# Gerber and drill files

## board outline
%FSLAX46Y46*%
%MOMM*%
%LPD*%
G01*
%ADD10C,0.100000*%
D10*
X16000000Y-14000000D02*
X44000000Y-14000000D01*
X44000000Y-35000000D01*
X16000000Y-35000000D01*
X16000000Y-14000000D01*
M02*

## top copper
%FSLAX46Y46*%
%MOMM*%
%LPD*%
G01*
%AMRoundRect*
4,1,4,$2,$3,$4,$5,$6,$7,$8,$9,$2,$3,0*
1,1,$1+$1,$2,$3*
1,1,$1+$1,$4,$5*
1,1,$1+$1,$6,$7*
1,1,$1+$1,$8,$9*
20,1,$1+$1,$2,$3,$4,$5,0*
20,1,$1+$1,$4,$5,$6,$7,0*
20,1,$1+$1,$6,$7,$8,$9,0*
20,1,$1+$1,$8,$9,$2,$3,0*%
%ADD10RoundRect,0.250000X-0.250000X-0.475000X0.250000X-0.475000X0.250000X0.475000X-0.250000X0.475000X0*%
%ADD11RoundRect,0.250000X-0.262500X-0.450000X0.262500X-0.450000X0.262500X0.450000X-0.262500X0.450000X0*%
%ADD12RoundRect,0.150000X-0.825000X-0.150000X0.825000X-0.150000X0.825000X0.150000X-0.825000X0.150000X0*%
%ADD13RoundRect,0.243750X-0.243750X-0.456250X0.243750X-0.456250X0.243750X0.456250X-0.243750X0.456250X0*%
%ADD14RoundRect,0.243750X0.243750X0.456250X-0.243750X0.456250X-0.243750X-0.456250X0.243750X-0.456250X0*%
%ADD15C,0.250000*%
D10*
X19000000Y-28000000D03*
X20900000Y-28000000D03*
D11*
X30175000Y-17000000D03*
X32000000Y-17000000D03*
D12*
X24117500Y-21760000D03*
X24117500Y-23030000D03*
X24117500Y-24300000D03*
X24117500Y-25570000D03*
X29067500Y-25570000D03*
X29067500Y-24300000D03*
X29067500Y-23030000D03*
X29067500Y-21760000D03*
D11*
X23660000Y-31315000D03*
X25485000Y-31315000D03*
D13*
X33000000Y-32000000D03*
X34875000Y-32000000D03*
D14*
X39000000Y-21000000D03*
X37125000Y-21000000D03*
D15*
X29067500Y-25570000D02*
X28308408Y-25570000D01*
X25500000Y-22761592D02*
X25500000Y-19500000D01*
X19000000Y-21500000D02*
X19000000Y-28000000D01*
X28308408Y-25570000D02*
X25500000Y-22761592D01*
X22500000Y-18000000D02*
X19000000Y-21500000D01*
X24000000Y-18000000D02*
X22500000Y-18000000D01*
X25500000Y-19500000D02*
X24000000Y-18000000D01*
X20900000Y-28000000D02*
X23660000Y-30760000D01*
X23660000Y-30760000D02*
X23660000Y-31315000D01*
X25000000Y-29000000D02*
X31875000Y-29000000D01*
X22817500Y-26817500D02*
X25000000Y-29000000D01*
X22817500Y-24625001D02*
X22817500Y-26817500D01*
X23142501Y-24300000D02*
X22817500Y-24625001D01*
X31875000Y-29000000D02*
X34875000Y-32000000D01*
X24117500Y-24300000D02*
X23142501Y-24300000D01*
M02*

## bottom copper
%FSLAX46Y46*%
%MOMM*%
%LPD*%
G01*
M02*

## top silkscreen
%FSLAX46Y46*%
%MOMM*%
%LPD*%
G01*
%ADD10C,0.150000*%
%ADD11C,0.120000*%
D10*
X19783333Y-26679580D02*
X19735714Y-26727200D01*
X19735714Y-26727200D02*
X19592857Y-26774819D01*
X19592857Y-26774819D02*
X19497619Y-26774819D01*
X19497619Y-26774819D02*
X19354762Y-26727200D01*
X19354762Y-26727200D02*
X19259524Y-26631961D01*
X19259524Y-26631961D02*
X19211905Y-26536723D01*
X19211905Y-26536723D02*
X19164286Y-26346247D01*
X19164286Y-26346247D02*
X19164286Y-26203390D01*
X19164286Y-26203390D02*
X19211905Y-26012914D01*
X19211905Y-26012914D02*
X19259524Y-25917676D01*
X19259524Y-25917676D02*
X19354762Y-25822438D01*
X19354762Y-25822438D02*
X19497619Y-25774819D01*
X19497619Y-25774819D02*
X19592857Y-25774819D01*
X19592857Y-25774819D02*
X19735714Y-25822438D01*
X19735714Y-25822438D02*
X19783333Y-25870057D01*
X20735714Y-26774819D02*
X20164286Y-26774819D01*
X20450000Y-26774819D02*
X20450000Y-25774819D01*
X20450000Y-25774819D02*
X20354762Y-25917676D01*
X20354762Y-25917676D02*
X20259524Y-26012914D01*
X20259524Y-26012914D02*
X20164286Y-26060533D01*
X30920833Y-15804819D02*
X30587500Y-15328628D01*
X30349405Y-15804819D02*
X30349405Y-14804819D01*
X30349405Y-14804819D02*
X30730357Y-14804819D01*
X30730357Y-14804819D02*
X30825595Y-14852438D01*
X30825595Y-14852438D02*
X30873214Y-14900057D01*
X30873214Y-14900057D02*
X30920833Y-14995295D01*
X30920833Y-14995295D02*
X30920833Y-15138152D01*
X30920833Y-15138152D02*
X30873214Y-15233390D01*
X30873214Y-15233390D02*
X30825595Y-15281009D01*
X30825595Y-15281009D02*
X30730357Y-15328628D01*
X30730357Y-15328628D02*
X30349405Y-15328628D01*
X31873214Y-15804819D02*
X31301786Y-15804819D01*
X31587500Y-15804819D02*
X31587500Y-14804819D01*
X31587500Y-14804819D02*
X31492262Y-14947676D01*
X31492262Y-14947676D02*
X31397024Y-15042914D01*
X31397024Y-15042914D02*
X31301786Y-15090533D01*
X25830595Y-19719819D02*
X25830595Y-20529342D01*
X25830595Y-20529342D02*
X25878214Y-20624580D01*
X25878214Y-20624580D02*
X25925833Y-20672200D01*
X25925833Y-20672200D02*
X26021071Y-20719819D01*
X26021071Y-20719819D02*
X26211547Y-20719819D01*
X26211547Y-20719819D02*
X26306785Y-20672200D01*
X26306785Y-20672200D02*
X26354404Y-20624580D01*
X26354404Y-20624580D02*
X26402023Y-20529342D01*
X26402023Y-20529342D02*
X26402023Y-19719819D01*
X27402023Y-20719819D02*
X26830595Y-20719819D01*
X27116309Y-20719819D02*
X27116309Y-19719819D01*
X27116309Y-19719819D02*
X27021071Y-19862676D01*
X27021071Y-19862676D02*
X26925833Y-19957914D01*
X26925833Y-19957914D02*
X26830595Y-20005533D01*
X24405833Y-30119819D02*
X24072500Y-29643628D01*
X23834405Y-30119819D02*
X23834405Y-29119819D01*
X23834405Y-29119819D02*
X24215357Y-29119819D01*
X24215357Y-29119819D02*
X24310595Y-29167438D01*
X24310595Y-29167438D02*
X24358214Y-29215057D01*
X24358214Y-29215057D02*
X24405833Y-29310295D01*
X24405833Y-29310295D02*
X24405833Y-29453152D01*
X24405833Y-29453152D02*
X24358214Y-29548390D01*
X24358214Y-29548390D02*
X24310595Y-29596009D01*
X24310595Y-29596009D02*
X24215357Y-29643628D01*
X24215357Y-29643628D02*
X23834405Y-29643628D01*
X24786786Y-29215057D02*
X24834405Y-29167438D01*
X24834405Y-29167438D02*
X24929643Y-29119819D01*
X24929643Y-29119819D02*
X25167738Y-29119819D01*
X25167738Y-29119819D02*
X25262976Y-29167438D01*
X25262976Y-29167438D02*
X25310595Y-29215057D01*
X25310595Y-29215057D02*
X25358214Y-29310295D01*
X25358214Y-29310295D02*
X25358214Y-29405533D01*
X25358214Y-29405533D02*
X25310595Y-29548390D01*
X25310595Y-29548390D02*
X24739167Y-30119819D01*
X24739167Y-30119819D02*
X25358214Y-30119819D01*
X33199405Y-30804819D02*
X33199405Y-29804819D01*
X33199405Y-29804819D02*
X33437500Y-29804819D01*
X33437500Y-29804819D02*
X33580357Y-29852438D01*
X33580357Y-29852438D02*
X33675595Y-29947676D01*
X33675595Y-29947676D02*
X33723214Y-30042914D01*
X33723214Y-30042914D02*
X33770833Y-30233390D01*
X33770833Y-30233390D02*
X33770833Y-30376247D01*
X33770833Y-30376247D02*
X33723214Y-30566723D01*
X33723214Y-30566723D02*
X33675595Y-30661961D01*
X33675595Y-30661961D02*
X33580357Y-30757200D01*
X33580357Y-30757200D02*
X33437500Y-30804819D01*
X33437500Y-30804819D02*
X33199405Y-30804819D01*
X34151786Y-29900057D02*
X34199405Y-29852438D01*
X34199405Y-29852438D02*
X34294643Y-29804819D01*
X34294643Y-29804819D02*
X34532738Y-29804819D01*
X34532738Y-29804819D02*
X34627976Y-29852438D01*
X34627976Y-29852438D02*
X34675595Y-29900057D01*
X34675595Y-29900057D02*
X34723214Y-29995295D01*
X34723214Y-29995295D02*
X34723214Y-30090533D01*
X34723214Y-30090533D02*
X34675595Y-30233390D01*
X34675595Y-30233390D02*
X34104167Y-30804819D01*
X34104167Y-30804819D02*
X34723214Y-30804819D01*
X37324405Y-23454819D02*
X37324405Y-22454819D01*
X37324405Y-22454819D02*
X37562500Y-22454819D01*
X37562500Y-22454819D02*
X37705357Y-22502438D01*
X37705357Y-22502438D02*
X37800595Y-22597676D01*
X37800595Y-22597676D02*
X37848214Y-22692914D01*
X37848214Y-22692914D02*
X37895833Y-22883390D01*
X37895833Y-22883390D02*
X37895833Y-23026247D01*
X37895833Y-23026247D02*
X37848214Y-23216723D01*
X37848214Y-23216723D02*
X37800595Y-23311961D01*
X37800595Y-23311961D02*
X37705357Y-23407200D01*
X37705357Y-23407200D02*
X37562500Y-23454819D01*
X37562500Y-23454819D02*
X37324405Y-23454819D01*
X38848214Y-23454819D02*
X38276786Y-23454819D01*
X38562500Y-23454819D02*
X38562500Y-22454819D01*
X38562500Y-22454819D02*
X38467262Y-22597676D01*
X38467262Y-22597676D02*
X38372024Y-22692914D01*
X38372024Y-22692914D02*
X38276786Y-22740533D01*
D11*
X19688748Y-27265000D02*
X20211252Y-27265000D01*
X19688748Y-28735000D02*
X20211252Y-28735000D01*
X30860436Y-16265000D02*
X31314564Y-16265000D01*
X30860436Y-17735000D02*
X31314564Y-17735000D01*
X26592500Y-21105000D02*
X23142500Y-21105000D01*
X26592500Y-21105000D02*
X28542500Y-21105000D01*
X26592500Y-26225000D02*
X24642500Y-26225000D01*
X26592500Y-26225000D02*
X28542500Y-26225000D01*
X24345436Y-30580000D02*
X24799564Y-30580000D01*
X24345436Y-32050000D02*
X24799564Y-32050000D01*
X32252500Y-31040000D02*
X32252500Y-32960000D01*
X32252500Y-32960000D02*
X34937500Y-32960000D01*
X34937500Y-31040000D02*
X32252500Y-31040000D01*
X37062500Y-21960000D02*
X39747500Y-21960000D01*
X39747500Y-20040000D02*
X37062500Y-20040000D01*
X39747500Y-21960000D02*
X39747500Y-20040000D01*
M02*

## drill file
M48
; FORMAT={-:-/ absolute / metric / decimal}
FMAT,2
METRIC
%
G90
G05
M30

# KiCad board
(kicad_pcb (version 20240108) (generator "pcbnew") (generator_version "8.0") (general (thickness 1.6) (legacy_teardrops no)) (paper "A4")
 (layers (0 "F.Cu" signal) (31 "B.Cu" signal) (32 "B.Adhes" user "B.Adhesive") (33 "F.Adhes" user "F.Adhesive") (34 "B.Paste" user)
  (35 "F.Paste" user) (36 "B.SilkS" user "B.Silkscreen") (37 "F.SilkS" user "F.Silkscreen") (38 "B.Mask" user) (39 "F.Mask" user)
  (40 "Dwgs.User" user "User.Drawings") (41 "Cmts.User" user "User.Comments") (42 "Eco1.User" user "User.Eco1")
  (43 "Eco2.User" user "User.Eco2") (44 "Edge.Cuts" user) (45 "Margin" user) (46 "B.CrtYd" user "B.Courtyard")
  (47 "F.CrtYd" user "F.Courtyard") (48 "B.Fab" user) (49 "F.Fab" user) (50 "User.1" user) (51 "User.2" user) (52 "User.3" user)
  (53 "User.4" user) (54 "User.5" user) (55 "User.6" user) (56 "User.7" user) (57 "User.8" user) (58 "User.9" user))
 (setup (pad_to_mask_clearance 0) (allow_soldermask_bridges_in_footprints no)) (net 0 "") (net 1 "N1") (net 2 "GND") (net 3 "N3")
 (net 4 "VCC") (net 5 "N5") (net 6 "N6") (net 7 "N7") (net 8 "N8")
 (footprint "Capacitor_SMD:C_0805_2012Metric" (layer "F.Cu") (at 19.95 28)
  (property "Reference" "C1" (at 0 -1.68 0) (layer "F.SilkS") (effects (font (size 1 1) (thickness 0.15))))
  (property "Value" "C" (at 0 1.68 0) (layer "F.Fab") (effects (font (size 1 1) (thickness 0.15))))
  (fp_line (start -0.261252 -0.735) (end 0.261252 -0.735) (stroke (width 0.12) (type solid)) (layer "F.SilkS"))
  (fp_line (start -0.261252 0.735) (end 0.261252 0.735) (stroke (width 0.12) (type solid)) (layer "F.SilkS"))
  (pad "1" smd roundrect (at -0.95 0) (size 1 1.45) (layers "F.Cu" "F.Paste" "F.Mask") (roundrect_rratio 0.25) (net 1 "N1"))
  (pad "2" smd roundrect (at 0.95 0) (size 1 1.45) (layers "F.Cu" "F.Paste" "F.Mask") (roundrect_rratio 0.25) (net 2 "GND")))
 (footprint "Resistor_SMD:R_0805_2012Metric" (layer "F.Cu") (at 31.0875 17)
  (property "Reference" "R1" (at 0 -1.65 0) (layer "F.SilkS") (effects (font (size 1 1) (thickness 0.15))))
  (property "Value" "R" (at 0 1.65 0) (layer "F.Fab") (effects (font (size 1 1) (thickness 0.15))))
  (fp_line (start -0.227064 -0.735) (end 0.227064 -0.735) (stroke (width 0.12) (type solid)) (layer "F.SilkS"))
  (fp_line (start -0.227064 0.735) (end 0.227064 0.735) (stroke (width 0.12) (type solid)) (layer "F.SilkS"))
  (pad "1" smd roundrect (at -0.9125 0) (size 1.025 1.4) (layers "F.Cu" "F.Paste" "F.Mask") (roundrect_rratio 0.243902) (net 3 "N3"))
  (pad "2" smd roundrect (at 0.9125 0) (size 1.025 1.4) (layers "F.Cu" "F.Paste" "F.Mask") (roundrect_rratio 0.243902) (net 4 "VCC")))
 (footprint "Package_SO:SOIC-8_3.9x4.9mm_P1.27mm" (layer "F.Cu") (at 26.5925 23.665)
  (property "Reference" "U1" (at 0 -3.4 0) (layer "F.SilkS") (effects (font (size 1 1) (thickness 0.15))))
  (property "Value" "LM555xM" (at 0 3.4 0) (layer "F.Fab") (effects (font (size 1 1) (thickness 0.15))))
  (fp_line (start 0 -2.56) (end -3.45 -2.56) (stroke (width 0.12) (type solid)) (layer "F.SilkS"))
  (fp_line (start 0 -2.56) (end 1.95 -2.56) (stroke (width 0.12) (type solid)) (layer "F.SilkS"))
  (fp_line (start 0 2.56) (end -1.95 2.56) (stroke (width 0.12) (type solid)) (layer "F.SilkS"))
  (fp_line (start 0 2.56) (end 1.95 2.56) (stroke (width 0.12) (type solid)) (layer "F.SilkS"))
  (pad "1" smd roundrect (at -2.475 -1.905) (size 1.95 0.6) (layers "F.Cu" "F.Paste" "F.Mask") (roundrect_rratio 0.25) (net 2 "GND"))
  (pad "2" smd roundrect (at -2.475 -0.635) (size 1.95 0.6) (layers "F.Cu" "F.Paste" "F.Mask") (roundrect_rratio 0.25) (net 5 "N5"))
  (pad "3" smd roundrect (at -2.475 0.635) (size 1.95 0.6) (layers "F.Cu" "F.Paste" "F.Mask") (roundrect_rratio 0.25) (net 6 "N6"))
  (pad "4" smd roundrect (at -2.475 1.905) (size 1.95 0.6) (layers "F.Cu" "F.Paste" "F.Mask") (roundrect_rratio 0.25) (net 4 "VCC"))
  (pad "5" smd roundrect (at 2.475 1.905) (size 1.95 0.6) (layers "F.Cu" "F.Paste" "F.Mask") (roundrect_rratio 0.25) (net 1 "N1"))
  (pad "6" smd roundrect (at 2.475 0.635) (size 1.95 0.6) (layers "F.Cu" "F.Paste" "F.Mask") (roundrect_rratio 0.25) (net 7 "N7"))
  (pad "7" smd roundrect (at 2.475 -0.635) (size 1.95 0.6) (layers "F.Cu" "F.Paste" "F.Mask") (roundrect_rratio 0.25) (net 7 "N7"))
  (pad "8" smd roundrect (at 2.475 -1.905) (size 1.95 0.6) (layers "F.Cu" "F.Paste" "F.Mask") (roundrect_rratio 0.25) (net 4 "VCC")))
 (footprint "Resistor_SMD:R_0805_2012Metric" (layer "F.Cu") (at 24.5725 31.315)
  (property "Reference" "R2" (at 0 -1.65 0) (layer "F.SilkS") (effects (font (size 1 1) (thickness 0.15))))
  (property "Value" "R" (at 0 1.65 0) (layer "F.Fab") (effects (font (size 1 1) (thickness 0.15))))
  (fp_line (start -0.227064 -0.735) (end 0.227064 -0.735) (stroke (width 0.12) (type solid)) (layer "F.SilkS"))
  (fp_line (start -0.227064 0.735) (end 0.227064 0.735) (stroke (width 0.12) (type solid)) (layer "F.SilkS"))
  (pad "1" smd roundrect (at -0.9125 0) (size 1.025 1.4) (layers "F.Cu" "F.Paste" "F.Mask") (roundrect_rratio 0.243902) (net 2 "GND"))
  (pad "2" smd roundrect (at 0.9125 0) (size 1.025 1.4) (layers "F.Cu" "F.Paste" "F.Mask") (roundrect_rratio 0.243902) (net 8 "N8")))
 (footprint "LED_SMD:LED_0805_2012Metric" (layer "F.Cu") (at 33.9375 32)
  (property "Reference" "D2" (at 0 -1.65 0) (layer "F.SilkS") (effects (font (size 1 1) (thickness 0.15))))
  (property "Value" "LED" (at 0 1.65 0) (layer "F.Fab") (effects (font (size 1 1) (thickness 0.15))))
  (fp_line (start -1.685 -0.96) (end -1.685 0.96) (stroke (width 0.12) (type solid)) (layer "F.SilkS"))
  (fp_line (start -1.685 0.96) (end 1 0.96) (stroke (width 0.12) (type solid)) (layer "F.SilkS"))
  (fp_line (start 1 -0.96) (end -1.685 -0.96) (stroke (width 0.12) (type solid)) (layer "F.SilkS"))
  (pad "1" smd roundrect (at -0.9375 0) (size 0.975 1.4) (layers "F.Cu" "F.Paste" "F.Mask") (roundrect_rratio 0.25) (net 8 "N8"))
  (pad "2" smd roundrect (at 0.9375 0) (size 0.975 1.4) (layers "F.Cu" "F.Paste" "F.Mask") (roundrect_rratio 0.25) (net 6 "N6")))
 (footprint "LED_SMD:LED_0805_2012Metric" (layer "F.Cu") (at 38.0625 21 180)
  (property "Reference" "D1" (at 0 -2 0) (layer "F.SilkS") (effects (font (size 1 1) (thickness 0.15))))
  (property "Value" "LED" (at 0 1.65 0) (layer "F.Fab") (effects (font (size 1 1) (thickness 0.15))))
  (fp_line (start 1 -0.96) (end -1.685 -0.96) (stroke (width 0.12) (type solid)) (layer "F.SilkS"))
  (fp_line (start -1.685 0.96) (end 1 0.96) (stroke (width 0.12) (type solid)) (layer "F.SilkS"))
  (fp_line (start -1.685 -0.96) (end -1.685 0.96) (stroke (width 0.12) (type solid)) (layer "F.SilkS"))
  (pad "1" smd roundrect (at -0.9375 0 180) (size 0.975 1.4) (layers "F.Cu" "F.Paste" "F.Mask") (roundrect_rratio 0.25) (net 6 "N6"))
  (pad "2" smd roundrect (at 0.9375 0 180) (size 0.975 1.4) (layers "F.Cu" "F.Paste" "F.Mask") (roundrect_rratio 0.25) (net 3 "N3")))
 (gr_rect (start 16 14) (end 44 35) (stroke (width 0.1) (type default)) (fill none) (layer "Edge.Cuts"))
 (segment (start 29.0675 25.57) (end 28.308408 25.57) (width 0.25) (layer "F.Cu") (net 1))
 (segment (start 25.5 22.761592) (end 25.5 19.5) (width 0.25) (layer "F.Cu") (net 1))
 (segment (start 19 21.5) (end 19 28) (width 0.25) (layer "F.Cu") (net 1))
 (segment (start 28.308408 25.57) (end 25.5 22.761592) (width 0.25) (layer "F.Cu") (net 1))
 (segment (start 22.5 18) (end 19 21.5) (width 0.25) (layer "F.Cu") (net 1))
 (segment (start 24 18) (end 22.5 18) (width 0.25) (layer "F.Cu") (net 1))
 (segment (start 25.5 19.5) (end 24 18) (width 0.25) (layer "F.Cu") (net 1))
 (segment (start 20.9 28) (end 23.66 30.76) (width 0.25) (layer "F.Cu") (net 2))
 (segment (start 23.66 30.76) (end 23.66 31.315) (width 0.25) (layer "F.Cu") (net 2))
 (segment (start 25 29) (end 31.875 29) (width 0.25) (layer "F.Cu") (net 6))
 (segment (start 22.8175 26.8175) (end 25 29) (width 0.25) (layer "F.Cu") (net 6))
 (segment (start 22.8175 24.625001) (end 22.8175 26.8175) (width 0.25) (layer "F.Cu") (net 6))
 (segment (start 23.142501 24.3) (end 22.8175 24.625001) (width 0.25) (layer "F.Cu") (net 6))
 (segment (start 31.875 29) (end 34.875 32) (width 0.25) (layer "F.Cu") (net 6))
 (segment (start 24.1175 24.3) (end 23.142501 24.3) (width 0.25) (layer "F.Cu") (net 6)))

